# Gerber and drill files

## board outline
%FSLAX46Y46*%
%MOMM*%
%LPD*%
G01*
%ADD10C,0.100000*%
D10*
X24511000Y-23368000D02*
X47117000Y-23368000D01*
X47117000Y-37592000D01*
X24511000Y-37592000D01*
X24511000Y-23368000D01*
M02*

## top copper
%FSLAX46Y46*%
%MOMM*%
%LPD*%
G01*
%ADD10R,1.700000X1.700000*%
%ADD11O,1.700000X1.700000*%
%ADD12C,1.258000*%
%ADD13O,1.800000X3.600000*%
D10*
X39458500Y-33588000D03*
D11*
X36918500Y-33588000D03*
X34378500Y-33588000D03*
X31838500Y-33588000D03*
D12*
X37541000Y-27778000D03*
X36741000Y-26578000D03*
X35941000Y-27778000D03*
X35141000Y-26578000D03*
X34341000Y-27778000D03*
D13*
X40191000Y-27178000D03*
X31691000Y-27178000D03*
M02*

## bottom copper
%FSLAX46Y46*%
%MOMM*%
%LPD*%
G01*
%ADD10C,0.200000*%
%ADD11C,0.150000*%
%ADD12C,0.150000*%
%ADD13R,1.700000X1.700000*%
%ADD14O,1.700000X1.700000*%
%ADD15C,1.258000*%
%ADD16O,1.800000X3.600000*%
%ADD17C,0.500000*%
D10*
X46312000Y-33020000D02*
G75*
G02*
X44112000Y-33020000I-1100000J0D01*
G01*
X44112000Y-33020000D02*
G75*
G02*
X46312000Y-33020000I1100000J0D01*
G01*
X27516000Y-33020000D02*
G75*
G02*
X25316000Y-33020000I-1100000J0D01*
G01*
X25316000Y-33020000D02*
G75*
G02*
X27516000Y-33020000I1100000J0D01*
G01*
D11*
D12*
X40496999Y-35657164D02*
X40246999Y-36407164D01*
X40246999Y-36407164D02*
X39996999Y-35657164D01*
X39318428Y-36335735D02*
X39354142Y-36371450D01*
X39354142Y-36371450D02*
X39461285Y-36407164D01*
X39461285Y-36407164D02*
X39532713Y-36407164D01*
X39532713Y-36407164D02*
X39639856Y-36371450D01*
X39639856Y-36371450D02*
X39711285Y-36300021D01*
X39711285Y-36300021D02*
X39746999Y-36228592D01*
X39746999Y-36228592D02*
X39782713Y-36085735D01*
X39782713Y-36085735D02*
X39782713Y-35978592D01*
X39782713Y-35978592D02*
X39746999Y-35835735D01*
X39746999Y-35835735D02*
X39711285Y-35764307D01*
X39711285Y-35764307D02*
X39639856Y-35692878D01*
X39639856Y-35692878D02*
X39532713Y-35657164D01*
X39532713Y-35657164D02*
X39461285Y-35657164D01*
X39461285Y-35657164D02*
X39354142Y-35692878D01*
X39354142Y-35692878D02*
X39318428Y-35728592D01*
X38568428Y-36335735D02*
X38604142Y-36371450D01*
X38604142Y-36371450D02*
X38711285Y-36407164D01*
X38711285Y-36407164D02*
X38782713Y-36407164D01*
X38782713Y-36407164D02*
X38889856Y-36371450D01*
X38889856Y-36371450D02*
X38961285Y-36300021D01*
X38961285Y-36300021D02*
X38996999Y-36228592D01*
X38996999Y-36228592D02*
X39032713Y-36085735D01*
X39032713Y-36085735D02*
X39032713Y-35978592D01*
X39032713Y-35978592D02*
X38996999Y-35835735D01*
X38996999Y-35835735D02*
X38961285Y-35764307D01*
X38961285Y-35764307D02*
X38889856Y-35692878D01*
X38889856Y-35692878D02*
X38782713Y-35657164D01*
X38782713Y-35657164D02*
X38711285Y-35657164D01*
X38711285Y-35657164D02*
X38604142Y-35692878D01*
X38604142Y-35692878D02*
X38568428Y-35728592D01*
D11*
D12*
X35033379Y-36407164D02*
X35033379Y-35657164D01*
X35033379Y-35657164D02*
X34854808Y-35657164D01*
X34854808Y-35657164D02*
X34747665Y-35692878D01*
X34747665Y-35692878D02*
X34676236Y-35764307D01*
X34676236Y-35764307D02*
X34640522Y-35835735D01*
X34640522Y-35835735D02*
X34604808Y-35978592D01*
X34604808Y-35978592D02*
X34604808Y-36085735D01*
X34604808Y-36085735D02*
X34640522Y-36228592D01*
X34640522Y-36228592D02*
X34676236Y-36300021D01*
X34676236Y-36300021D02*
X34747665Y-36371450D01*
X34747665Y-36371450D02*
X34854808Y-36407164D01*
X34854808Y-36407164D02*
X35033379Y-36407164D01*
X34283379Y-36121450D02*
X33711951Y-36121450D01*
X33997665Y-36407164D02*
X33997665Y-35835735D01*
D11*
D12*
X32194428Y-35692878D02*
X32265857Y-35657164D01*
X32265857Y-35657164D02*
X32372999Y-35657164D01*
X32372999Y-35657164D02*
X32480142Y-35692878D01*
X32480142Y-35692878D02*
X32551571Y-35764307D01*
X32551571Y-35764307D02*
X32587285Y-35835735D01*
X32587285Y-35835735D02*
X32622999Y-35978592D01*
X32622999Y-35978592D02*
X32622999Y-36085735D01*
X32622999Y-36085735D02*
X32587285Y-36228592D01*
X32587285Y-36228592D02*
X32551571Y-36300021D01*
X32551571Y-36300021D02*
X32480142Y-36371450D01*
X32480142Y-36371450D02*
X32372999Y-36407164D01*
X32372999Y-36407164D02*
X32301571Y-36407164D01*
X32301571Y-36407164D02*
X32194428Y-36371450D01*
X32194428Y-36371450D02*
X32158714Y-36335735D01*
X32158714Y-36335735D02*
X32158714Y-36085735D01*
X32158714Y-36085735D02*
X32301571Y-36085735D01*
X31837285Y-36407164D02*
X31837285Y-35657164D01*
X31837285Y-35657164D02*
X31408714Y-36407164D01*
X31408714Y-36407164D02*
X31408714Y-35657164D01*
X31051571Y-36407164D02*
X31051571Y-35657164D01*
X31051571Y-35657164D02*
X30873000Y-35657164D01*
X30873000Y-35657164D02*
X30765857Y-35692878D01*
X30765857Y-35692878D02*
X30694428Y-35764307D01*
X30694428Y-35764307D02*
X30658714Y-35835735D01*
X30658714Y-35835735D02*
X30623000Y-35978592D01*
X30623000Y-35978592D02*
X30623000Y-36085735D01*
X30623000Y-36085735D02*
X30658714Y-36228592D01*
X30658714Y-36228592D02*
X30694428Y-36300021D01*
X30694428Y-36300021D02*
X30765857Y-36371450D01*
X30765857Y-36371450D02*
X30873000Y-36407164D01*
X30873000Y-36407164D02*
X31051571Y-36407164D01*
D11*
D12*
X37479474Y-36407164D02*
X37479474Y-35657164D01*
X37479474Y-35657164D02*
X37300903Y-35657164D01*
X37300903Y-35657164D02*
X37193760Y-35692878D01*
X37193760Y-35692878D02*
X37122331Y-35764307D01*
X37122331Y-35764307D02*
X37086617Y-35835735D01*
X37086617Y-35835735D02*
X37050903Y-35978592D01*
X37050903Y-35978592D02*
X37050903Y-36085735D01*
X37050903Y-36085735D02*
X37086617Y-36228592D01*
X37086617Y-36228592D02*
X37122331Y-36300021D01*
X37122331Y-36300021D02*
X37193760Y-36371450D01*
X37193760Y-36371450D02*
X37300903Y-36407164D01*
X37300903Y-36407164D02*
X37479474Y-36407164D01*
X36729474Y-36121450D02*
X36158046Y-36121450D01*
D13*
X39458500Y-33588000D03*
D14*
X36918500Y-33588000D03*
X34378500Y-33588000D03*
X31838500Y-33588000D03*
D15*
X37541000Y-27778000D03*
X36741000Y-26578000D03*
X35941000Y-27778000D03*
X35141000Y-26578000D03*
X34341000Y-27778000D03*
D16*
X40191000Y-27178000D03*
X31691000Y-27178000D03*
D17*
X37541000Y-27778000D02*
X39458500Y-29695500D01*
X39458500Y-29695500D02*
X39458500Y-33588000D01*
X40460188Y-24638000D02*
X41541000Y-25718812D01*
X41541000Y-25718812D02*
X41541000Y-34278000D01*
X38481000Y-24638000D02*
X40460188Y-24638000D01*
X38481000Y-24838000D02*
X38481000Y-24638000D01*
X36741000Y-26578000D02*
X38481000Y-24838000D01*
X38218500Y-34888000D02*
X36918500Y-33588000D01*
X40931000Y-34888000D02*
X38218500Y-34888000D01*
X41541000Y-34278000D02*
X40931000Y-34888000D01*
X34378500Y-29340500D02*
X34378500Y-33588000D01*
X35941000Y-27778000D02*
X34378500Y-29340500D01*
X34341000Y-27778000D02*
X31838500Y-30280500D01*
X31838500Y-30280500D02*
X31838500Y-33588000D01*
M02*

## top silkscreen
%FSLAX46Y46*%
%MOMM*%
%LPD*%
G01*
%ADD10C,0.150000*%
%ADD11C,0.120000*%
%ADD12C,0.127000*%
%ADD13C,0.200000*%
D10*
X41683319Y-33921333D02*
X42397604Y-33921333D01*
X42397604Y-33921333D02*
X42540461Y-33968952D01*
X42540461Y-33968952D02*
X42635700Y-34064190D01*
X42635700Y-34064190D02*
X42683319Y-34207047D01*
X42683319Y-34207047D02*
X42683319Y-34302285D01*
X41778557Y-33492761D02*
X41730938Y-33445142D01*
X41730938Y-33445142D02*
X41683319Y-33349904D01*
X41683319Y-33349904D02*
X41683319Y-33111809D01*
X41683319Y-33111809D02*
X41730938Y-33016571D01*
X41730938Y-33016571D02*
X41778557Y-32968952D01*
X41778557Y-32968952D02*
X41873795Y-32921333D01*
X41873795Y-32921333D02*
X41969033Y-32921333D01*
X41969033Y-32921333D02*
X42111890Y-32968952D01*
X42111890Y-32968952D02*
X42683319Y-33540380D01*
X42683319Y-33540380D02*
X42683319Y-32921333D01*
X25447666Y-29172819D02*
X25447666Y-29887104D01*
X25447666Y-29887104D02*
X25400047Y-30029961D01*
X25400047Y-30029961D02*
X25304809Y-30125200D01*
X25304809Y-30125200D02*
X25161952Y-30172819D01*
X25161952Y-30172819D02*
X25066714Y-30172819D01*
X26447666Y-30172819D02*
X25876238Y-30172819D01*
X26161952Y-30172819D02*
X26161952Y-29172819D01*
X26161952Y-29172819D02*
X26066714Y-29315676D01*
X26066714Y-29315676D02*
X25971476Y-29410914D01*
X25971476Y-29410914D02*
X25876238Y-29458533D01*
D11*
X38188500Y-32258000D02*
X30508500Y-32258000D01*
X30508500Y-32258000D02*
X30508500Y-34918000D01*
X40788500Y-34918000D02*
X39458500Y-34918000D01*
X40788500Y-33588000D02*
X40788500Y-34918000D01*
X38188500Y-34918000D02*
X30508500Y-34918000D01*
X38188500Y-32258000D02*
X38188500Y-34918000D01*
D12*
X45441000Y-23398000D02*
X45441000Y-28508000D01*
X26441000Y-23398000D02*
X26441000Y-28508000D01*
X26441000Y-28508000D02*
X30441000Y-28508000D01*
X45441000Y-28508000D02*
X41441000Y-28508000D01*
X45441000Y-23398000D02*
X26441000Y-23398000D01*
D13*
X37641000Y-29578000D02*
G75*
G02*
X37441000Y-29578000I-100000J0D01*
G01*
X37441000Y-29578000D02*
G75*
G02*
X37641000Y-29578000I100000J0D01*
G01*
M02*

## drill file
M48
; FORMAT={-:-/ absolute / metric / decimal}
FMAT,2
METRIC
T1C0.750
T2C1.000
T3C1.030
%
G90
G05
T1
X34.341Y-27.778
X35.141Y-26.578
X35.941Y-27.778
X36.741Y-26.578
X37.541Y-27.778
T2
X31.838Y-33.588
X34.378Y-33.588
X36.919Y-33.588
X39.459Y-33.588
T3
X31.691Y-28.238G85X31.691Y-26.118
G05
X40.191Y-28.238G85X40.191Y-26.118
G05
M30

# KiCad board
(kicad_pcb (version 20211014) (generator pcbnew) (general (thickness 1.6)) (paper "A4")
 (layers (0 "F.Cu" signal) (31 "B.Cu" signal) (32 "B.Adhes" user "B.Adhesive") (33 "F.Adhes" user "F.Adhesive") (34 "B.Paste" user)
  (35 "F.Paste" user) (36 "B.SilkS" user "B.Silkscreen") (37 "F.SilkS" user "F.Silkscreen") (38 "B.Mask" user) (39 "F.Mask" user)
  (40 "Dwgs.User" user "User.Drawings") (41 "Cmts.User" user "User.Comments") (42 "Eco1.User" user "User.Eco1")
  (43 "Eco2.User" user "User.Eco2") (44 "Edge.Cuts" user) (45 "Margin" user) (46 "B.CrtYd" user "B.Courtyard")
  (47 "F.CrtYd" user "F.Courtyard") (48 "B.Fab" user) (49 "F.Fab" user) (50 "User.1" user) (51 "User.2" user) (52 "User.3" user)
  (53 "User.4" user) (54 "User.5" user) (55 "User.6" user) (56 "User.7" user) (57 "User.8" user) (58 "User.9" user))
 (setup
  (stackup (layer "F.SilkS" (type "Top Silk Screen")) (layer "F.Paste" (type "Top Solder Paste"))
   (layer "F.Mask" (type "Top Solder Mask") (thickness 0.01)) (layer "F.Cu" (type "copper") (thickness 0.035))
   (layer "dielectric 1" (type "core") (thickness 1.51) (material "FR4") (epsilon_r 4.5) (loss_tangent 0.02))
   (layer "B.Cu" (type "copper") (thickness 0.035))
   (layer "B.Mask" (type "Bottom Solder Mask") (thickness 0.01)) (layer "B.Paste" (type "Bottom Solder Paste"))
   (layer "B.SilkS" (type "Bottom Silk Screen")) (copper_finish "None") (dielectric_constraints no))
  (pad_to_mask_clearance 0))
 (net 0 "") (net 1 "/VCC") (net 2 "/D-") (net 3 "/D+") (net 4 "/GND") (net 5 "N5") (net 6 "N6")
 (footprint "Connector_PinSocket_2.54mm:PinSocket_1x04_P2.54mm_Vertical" (layer "F.Cu") (at 39.4585 33.588 -90)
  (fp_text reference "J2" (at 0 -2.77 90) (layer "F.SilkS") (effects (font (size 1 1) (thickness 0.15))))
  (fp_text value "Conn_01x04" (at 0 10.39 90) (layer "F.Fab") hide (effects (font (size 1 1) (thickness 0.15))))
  (fp_line (start -1.33 1.27) (end -1.33 8.95) (layer "F.SilkS") (width 0.12))
  (fp_line (start -1.33 8.95) (end 1.33 8.95) (layer "F.SilkS") (width 0.12))
  (fp_line (start 1.33 -1.33) (end 1.33 0) (layer "F.SilkS") (width 0.12))
  (fp_line (start 0 -1.33) (end 1.33 -1.33) (layer "F.SilkS") (width 0.12))
  (fp_line (start 1.33 1.27) (end 1.33 8.95) (layer "F.SilkS") (width 0.12))
  (fp_line (start -1.33 1.27) (end 1.33 1.27) (layer "F.SilkS") (width 0.12))
  (pad "1" thru_hole rect (at 0 0 270) (size 1.7 1.7) (drill 1) (layers *.Cu *.Mask) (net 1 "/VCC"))
  (pad "2" thru_hole oval (at 0 2.54 270) (size 1.7 1.7) (drill 1) (layers *.Cu *.Mask) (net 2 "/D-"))
  (pad "3" thru_hole oval (at 0 5.08 270) (size 1.7 1.7) (drill 1) (layers *.Cu *.Mask) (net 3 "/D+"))
  (pad "4" thru_hole oval (at 0 7.62 270) (size 1.7 1.7) (drill 1) (layers *.Cu *.Mask) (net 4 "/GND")))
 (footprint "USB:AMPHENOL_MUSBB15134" (layer "F.Cu") (at 35.941 27.178 180)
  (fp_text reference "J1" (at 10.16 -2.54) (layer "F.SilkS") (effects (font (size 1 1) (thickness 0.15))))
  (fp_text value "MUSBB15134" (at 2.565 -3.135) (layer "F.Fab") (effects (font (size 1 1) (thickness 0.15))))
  (fp_line (start -9.5 3.78) (end -9.5 -1.33) (layer "F.SilkS") (width 0.127))
  (fp_line (start 9.5 3.78) (end 9.5 -1.33) (layer "F.SilkS") (width 0.127))
  (fp_line (start 9.5 -1.33) (end 5.5 -1.33) (layer "F.SilkS") (width 0.127))
  (fp_line (start -9.5 -1.33) (end -5.5 -1.33) (layer "F.SilkS") (width 0.127))
  (fp_line (start -9.5 3.78) (end 9.5 3.78) (layer "F.SilkS") (width 0.127))
  (fp_circle (center -1.6 -2.4) (end -1.5 -2.4) (layer "F.SilkS") (width 0.2) (fill none))
  (pad "1" thru_hole circle (at -1.6 -0.6 180) (size 1.258 1.258) (drill 0.75) (layers *.Cu *.Mask) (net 1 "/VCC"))
  (pad "2" thru_hole circle (at -0.8 0.6 180) (size 1.258 1.258) (drill 0.75) (layers *.Cu *.Mask) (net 2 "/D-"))
  (pad "3" thru_hole circle (at 0 -0.6 180) (size 1.258 1.258) (drill 0.75) (layers *.Cu *.Mask) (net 3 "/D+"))
  (pad "4" thru_hole circle (at 0.8 0.6 180) (size 1.258 1.258) (drill 0.75) (layers *.Cu *.Mask) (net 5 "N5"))
  (pad "5" thru_hole circle (at 1.6 -0.6 180) (size 1.258 1.258) (drill 0.75) (layers *.Cu *.Mask) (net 4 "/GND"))
  (pad "S1" thru_hole oval (at -4.25 0 180) (size 1.8 3.6) (drill oval 1.03 3.15) (layers *.Cu *.Mask) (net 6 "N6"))
  (pad "S2" thru_hole oval (at 4.25 0 180) (size 1.8 3.6) (drill oval 1.03 3.15) (layers *.Cu *.Mask) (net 6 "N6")))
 (gr_circle (center 45.212 33.02) (end 46.312 33.02) (layer "B.Cu") (width 0.2) (fill none))
 (gr_circle (center 26.416 33.02) (end 27.516 33.02) (layer "B.Cu") (width 0.2) (fill none))
 (gr_rect (start 24.511 37.592) (end 47.117 23.368) (layer "Edge.Cuts") (width 0.1) (fill none))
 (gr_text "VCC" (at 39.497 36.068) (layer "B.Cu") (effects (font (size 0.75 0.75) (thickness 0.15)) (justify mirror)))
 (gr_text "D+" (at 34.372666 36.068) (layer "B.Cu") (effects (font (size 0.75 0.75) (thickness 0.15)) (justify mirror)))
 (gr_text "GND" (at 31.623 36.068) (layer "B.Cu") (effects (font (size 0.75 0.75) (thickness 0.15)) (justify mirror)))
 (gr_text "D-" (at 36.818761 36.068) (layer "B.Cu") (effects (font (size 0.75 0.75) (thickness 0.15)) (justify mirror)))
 (segment (start 37.541 27.778) (end 39.4585 29.6955) (width 0.5) (layer "B.Cu") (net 1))
 (segment (start 39.4585 29.6955) (end 39.4585 33.588) (width 0.5) (layer "B.Cu") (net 1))
 (segment (start 40.460188 24.638) (end 41.541 25.718812) (width 0.5) (layer "B.Cu") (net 2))
 (segment (start 41.541 25.718812) (end 41.541 34.278) (width 0.5) (layer "B.Cu") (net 2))
 (segment (start 38.481 24.638) (end 40.460188 24.638) (width 0.5) (layer "B.Cu") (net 2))
 (segment (start 38.481 24.838) (end 38.481 24.638) (width 0.5) (layer "B.Cu") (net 2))
 (segment (start 36.741 26.578) (end 38.481 24.838) (width 0.5) (layer "B.Cu") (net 2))
 (segment (start 38.2185 34.888) (end 36.9185 33.588) (width 0.5) (layer "B.Cu") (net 2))
 (segment (start 40.931 34.888) (end 38.2185 34.888) (width 0.5) (layer "B.Cu") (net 2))
 (segment (start 41.541 34.278) (end 40.931 34.888) (width 0.5) (layer "B.Cu") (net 2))
 (segment (start 34.3785 29.3405) (end 34.3785 33.588) (width 0.5) (layer "B.Cu") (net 3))
 (segment (start 35.941 27.778) (end 34.3785 29.3405) (width 0.5) (layer "B.Cu") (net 3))
 (segment (start 34.341 27.778) (end 31.8385 30.2805) (width 0.5) (layer "B.Cu") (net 4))
 (segment (start 31.8385 30.2805) (end 31.8385 33.588) (width 0.5) (layer "B.Cu") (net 4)))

